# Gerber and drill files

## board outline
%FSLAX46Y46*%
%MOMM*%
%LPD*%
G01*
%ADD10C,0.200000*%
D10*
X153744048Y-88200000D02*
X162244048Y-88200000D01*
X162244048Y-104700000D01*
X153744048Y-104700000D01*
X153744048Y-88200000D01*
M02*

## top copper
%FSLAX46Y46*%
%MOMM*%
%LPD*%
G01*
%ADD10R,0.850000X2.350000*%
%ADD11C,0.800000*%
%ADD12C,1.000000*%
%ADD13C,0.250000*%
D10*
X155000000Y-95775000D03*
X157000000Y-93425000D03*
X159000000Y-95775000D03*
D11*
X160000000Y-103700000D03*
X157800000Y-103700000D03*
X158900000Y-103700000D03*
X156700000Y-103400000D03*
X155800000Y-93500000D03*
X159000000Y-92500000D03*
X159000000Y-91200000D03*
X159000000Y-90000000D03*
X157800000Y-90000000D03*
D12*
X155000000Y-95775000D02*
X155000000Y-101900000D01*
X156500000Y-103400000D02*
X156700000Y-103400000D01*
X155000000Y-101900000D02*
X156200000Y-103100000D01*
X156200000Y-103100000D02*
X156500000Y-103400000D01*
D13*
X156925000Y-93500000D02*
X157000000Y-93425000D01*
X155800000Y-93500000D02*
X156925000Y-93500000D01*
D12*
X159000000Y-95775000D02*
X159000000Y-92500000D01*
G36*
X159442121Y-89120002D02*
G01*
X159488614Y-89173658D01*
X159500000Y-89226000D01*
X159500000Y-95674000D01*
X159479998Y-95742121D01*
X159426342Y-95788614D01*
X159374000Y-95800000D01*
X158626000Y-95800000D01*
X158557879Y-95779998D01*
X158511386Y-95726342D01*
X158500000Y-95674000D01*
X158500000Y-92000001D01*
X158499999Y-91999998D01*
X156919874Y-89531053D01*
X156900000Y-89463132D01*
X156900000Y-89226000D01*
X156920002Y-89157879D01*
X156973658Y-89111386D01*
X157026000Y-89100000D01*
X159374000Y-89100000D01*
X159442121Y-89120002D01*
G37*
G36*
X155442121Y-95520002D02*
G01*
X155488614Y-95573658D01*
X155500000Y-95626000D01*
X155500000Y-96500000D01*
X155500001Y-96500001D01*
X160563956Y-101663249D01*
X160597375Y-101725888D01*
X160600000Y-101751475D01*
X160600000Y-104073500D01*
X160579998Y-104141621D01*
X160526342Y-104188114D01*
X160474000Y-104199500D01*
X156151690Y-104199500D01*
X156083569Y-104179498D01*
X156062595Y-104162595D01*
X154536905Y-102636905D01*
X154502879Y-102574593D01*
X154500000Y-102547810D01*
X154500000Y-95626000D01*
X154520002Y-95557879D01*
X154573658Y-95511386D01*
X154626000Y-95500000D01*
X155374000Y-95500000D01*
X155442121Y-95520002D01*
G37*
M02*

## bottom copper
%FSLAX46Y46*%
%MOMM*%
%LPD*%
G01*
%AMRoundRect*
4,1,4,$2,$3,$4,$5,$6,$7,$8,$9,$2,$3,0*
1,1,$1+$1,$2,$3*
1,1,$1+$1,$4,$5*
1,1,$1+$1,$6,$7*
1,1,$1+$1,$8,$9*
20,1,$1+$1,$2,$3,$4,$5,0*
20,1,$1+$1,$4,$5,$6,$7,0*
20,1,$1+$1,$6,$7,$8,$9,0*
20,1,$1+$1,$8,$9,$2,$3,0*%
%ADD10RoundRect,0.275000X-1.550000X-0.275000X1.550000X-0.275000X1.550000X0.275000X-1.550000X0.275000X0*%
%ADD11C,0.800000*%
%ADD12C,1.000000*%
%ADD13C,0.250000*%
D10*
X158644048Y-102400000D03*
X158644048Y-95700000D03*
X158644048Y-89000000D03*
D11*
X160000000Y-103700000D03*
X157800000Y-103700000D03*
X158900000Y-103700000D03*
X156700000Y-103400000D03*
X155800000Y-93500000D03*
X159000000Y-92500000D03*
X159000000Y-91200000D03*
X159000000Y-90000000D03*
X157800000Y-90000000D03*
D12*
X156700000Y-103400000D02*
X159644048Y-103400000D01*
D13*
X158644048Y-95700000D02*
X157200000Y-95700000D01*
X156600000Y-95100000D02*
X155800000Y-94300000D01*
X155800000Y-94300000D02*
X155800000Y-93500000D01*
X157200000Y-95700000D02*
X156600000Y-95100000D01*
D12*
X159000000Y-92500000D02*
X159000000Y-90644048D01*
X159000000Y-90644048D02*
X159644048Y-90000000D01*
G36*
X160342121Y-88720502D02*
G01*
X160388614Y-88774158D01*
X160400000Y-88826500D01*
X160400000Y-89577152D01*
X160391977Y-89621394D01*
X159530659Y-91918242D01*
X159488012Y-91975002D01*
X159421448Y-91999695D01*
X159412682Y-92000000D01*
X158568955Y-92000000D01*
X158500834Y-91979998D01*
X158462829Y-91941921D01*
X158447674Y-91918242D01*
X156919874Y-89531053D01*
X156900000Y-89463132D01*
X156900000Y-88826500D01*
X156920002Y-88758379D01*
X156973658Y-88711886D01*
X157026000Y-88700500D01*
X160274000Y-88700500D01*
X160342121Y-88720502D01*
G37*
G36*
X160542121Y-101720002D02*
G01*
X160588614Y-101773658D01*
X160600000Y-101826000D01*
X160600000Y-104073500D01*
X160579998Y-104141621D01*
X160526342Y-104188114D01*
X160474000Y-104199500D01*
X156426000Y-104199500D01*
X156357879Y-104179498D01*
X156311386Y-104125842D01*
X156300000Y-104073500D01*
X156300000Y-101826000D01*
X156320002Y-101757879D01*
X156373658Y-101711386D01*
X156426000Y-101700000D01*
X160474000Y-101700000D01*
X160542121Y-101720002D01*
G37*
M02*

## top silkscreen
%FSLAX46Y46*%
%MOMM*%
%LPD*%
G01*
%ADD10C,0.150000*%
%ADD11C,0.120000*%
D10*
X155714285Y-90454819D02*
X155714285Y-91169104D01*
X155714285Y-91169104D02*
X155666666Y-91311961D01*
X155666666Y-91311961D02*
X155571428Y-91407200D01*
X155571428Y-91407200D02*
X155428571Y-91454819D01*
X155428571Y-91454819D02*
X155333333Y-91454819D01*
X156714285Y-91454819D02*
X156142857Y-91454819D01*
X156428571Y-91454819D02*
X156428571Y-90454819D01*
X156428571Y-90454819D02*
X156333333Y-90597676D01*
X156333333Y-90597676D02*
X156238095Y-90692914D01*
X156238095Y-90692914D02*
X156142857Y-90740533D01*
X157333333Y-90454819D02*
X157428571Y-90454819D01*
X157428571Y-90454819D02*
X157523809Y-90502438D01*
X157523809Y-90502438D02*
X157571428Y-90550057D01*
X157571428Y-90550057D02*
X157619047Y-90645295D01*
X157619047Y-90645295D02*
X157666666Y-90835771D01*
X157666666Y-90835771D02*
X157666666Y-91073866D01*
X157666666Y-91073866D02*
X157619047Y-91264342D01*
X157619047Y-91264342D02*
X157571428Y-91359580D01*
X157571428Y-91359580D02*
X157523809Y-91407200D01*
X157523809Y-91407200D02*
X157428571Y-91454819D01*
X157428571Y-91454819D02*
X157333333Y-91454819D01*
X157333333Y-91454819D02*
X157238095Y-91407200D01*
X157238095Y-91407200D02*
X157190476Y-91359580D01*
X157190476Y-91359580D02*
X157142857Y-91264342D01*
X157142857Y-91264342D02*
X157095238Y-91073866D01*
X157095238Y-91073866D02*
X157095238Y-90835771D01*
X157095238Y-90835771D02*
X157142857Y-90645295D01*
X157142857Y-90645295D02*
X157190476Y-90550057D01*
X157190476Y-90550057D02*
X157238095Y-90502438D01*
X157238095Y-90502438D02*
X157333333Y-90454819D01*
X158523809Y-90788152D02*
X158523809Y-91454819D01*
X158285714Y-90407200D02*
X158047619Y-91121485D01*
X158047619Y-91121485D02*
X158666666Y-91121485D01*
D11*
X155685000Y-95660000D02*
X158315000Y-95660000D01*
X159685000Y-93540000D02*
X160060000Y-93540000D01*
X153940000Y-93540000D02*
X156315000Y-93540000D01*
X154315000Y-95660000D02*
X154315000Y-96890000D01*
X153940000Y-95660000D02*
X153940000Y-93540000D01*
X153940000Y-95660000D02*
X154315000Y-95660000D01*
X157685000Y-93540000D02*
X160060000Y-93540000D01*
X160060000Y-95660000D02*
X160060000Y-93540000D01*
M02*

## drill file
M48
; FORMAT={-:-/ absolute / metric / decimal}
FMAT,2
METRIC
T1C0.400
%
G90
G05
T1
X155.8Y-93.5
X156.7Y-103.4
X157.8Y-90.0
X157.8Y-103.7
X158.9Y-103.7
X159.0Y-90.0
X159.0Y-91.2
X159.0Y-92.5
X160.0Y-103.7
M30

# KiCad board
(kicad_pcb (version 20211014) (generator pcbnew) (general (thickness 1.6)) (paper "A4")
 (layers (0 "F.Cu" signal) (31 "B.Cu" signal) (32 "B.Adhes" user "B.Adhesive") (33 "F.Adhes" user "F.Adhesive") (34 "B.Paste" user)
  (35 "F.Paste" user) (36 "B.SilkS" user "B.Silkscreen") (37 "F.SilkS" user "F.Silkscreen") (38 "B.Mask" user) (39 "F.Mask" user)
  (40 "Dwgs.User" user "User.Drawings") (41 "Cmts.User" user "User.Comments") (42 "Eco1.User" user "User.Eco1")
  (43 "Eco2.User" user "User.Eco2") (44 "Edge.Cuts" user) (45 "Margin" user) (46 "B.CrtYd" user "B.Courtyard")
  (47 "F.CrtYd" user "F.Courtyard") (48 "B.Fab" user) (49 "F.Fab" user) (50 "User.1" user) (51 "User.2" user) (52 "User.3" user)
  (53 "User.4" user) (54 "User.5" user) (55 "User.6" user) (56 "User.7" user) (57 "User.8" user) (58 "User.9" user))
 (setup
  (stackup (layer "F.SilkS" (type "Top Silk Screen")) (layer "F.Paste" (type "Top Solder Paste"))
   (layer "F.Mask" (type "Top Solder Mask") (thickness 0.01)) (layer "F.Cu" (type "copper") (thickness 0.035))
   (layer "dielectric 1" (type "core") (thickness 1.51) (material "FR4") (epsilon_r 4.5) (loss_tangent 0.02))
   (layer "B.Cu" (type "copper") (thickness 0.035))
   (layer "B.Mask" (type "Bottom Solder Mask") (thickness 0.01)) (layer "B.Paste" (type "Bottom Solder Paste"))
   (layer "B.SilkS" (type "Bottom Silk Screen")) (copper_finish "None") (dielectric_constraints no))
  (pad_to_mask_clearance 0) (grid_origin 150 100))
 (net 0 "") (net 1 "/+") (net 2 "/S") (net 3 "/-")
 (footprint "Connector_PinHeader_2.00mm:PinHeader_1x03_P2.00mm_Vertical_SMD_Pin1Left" (layer "F.Cu") (at 157 94.6 90)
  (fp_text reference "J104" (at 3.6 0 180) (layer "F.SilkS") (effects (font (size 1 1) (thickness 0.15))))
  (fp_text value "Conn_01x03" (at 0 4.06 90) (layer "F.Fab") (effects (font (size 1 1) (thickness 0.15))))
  (fp_line (start -1.06 -1.315) (end -1.06 1.315) (layer "F.SilkS") (width 0.12))
  (fp_line (start 1.06 2.685) (end 1.06 3.06) (layer "F.SilkS") (width 0.12))
  (fp_line (start 1.06 -3.06) (end 1.06 -0.685) (layer "F.SilkS") (width 0.12))
  (fp_line (start -1.06 -2.685) (end -2.29 -2.685) (layer "F.SilkS") (width 0.12))
  (fp_line (start -1.06 -3.06) (end 1.06 -3.06) (layer "F.SilkS") (width 0.12))
  (fp_line (start -1.06 -3.06) (end -1.06 -2.685) (layer "F.SilkS") (width 0.12))
  (fp_line (start 1.06 0.685) (end 1.06 3.06) (layer "F.SilkS") (width 0.12))
  (fp_line (start -1.06 3.06) (end 1.06 3.06) (layer "F.SilkS") (width 0.12))
  (pad "1" smd rect (at -1.175 -2 90) (size 2.35 0.85) (layers "F.Cu" "F.Paste" "F.Mask") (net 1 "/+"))
  (pad "2" smd rect (at 1.175 0 90) (size 2.35 0.85) (layers "F.Cu" "F.Paste" "F.Mask") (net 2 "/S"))
  (pad "3" smd rect (at -1.175 2 90) (size 2.35 0.85) (layers "F.Cu" "F.Paste" "F.Mask") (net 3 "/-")))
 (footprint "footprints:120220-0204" (layer "B.Cu") (at 158.644048 102.4)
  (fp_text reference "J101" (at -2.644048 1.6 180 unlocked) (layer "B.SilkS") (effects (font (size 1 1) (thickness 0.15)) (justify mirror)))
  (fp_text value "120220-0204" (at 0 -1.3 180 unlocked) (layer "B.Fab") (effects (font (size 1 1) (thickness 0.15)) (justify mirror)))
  (pad "1" smd roundrect (at 0 0) (size 3.65 1.1) (layers "B.Cu" "B.Paste" "B.Mask") (roundrect_rratio 0.25) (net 1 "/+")))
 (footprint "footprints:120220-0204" (layer "B.Cu") (at 158.644048 95.7)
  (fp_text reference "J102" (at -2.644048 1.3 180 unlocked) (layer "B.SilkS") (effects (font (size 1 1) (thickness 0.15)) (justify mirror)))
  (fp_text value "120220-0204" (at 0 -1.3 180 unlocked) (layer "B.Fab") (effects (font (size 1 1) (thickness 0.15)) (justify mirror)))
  (pad "1" smd roundrect (at 0 0) (size 3.65 1.1) (layers "B.Cu" "B.Paste" "B.Mask") (roundrect_rratio 0.25) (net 2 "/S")))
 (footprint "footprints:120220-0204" (layer "B.Cu") (at 158.644048 89)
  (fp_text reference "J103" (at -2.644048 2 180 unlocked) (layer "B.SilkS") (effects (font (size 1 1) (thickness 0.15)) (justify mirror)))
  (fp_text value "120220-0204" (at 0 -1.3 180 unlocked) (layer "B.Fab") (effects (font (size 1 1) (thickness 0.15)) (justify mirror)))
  (pad "1" smd roundrect (at 0 0) (size 3.65 1.1) (layers "B.Cu" "B.Paste" "B.Mask") (roundrect_rratio 0.25) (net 3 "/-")))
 (gr_rect (start 153.744048 88.2) (end 162.244048 104.7) (layer "Edge.Cuts") (width 0.2) (fill none))
 (segment (start 155 95.775) (end 155 101.9) (width 1) (layer "F.Cu") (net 1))
 (segment (start 156.5 103.4) (end 156.7 103.4) (width 1) (layer "F.Cu") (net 1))
 (segment (start 155 101.9) (end 156.2 103.1) (width 1) (layer "F.Cu") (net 1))
 (segment (start 156.2 103.1) (end 156.5 103.4) (width 1) (layer "F.Cu") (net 1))
 (via (at 160 103.7) (size 0.8) (drill 0.4) (layers "F.Cu" "B.Cu") (free) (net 1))
 (via (at 157.8 103.7) (size 0.8) (drill 0.4) (layers "F.Cu" "B.Cu") (free) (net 1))
 (via (at 158.9 103.7) (size 0.8) (drill 0.4) (layers "F.Cu" "B.Cu") (free) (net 1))
 (via (at 156.7 103.4) (size 0.8) (drill 0.4) (layers "F.Cu" "B.Cu") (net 1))
 (segment (start 156.7 103.4) (end 159.644048 103.4) (width 1) (layer "B.Cu") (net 1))
 (segment (start 156.925 93.5) (end 157 93.425) (width 0.25) (layer "F.Cu") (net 2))
 (segment (start 155.8 93.5) (end 156.925 93.5) (width 0.25) (layer "F.Cu") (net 2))
 (via (at 155.8 93.5) (size 0.8) (drill 0.4) (layers "F.Cu" "B.Cu") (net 2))
 (segment (start 158.644048 95.7) (end 157.2 95.7) (width 0.25) (layer "B.Cu") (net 2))
 (segment (start 156.6 95.1) (end 155.8 94.3) (width 0.25) (layer "B.Cu") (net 2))
 (segment (start 155.8 94.3) (end 155.8 93.5) (width 0.25) (layer "B.Cu") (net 2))
 (segment (start 157.2 95.7) (end 156.6 95.1) (width 0.25) (layer "B.Cu") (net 2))
 (segment (start 159 95.775) (end 159 92.5) (width 1) (layer "F.Cu") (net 3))
 (via (at 159 92.5) (size 0.8) (drill 0.4) (layers "F.Cu" "B.Cu") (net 3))
 (via (at 159 91.2) (size 0.8) (drill 0.4) (layers "F.Cu" "B.Cu") (free) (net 3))
 (via (at 159 90) (size 0.8) (drill 0.4) (layers "F.Cu" "B.Cu") (free) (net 3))
 (via (at 157.8 90) (size 0.8) (drill 0.4) (layers "F.Cu" "B.Cu") (free) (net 3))
 (segment (start 159 92.5) (end 159 90.644048) (width 1) (layer "B.Cu") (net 3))
 (segment (start 159 90.644048) (end 159.644048 90) (width 1) (layer "B.Cu") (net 3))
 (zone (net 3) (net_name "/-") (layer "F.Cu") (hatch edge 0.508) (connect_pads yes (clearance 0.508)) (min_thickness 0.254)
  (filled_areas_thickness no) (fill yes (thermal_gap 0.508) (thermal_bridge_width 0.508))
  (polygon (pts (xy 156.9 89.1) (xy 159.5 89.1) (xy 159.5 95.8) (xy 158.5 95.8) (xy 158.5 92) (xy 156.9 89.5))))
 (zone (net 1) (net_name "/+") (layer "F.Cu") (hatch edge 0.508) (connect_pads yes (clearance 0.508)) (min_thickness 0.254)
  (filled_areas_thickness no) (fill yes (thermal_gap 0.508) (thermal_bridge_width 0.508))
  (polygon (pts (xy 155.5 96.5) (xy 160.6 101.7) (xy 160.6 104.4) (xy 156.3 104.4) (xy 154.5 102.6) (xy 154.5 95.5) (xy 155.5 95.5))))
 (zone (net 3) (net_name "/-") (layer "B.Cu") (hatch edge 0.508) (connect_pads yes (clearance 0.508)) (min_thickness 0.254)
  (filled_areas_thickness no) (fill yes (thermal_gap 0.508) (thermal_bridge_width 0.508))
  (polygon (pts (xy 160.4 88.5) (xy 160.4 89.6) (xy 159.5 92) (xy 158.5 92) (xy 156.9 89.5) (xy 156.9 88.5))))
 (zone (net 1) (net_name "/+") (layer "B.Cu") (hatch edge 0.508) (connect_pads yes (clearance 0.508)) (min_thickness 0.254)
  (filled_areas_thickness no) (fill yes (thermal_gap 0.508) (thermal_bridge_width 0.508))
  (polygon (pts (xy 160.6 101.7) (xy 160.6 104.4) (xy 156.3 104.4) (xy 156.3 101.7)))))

